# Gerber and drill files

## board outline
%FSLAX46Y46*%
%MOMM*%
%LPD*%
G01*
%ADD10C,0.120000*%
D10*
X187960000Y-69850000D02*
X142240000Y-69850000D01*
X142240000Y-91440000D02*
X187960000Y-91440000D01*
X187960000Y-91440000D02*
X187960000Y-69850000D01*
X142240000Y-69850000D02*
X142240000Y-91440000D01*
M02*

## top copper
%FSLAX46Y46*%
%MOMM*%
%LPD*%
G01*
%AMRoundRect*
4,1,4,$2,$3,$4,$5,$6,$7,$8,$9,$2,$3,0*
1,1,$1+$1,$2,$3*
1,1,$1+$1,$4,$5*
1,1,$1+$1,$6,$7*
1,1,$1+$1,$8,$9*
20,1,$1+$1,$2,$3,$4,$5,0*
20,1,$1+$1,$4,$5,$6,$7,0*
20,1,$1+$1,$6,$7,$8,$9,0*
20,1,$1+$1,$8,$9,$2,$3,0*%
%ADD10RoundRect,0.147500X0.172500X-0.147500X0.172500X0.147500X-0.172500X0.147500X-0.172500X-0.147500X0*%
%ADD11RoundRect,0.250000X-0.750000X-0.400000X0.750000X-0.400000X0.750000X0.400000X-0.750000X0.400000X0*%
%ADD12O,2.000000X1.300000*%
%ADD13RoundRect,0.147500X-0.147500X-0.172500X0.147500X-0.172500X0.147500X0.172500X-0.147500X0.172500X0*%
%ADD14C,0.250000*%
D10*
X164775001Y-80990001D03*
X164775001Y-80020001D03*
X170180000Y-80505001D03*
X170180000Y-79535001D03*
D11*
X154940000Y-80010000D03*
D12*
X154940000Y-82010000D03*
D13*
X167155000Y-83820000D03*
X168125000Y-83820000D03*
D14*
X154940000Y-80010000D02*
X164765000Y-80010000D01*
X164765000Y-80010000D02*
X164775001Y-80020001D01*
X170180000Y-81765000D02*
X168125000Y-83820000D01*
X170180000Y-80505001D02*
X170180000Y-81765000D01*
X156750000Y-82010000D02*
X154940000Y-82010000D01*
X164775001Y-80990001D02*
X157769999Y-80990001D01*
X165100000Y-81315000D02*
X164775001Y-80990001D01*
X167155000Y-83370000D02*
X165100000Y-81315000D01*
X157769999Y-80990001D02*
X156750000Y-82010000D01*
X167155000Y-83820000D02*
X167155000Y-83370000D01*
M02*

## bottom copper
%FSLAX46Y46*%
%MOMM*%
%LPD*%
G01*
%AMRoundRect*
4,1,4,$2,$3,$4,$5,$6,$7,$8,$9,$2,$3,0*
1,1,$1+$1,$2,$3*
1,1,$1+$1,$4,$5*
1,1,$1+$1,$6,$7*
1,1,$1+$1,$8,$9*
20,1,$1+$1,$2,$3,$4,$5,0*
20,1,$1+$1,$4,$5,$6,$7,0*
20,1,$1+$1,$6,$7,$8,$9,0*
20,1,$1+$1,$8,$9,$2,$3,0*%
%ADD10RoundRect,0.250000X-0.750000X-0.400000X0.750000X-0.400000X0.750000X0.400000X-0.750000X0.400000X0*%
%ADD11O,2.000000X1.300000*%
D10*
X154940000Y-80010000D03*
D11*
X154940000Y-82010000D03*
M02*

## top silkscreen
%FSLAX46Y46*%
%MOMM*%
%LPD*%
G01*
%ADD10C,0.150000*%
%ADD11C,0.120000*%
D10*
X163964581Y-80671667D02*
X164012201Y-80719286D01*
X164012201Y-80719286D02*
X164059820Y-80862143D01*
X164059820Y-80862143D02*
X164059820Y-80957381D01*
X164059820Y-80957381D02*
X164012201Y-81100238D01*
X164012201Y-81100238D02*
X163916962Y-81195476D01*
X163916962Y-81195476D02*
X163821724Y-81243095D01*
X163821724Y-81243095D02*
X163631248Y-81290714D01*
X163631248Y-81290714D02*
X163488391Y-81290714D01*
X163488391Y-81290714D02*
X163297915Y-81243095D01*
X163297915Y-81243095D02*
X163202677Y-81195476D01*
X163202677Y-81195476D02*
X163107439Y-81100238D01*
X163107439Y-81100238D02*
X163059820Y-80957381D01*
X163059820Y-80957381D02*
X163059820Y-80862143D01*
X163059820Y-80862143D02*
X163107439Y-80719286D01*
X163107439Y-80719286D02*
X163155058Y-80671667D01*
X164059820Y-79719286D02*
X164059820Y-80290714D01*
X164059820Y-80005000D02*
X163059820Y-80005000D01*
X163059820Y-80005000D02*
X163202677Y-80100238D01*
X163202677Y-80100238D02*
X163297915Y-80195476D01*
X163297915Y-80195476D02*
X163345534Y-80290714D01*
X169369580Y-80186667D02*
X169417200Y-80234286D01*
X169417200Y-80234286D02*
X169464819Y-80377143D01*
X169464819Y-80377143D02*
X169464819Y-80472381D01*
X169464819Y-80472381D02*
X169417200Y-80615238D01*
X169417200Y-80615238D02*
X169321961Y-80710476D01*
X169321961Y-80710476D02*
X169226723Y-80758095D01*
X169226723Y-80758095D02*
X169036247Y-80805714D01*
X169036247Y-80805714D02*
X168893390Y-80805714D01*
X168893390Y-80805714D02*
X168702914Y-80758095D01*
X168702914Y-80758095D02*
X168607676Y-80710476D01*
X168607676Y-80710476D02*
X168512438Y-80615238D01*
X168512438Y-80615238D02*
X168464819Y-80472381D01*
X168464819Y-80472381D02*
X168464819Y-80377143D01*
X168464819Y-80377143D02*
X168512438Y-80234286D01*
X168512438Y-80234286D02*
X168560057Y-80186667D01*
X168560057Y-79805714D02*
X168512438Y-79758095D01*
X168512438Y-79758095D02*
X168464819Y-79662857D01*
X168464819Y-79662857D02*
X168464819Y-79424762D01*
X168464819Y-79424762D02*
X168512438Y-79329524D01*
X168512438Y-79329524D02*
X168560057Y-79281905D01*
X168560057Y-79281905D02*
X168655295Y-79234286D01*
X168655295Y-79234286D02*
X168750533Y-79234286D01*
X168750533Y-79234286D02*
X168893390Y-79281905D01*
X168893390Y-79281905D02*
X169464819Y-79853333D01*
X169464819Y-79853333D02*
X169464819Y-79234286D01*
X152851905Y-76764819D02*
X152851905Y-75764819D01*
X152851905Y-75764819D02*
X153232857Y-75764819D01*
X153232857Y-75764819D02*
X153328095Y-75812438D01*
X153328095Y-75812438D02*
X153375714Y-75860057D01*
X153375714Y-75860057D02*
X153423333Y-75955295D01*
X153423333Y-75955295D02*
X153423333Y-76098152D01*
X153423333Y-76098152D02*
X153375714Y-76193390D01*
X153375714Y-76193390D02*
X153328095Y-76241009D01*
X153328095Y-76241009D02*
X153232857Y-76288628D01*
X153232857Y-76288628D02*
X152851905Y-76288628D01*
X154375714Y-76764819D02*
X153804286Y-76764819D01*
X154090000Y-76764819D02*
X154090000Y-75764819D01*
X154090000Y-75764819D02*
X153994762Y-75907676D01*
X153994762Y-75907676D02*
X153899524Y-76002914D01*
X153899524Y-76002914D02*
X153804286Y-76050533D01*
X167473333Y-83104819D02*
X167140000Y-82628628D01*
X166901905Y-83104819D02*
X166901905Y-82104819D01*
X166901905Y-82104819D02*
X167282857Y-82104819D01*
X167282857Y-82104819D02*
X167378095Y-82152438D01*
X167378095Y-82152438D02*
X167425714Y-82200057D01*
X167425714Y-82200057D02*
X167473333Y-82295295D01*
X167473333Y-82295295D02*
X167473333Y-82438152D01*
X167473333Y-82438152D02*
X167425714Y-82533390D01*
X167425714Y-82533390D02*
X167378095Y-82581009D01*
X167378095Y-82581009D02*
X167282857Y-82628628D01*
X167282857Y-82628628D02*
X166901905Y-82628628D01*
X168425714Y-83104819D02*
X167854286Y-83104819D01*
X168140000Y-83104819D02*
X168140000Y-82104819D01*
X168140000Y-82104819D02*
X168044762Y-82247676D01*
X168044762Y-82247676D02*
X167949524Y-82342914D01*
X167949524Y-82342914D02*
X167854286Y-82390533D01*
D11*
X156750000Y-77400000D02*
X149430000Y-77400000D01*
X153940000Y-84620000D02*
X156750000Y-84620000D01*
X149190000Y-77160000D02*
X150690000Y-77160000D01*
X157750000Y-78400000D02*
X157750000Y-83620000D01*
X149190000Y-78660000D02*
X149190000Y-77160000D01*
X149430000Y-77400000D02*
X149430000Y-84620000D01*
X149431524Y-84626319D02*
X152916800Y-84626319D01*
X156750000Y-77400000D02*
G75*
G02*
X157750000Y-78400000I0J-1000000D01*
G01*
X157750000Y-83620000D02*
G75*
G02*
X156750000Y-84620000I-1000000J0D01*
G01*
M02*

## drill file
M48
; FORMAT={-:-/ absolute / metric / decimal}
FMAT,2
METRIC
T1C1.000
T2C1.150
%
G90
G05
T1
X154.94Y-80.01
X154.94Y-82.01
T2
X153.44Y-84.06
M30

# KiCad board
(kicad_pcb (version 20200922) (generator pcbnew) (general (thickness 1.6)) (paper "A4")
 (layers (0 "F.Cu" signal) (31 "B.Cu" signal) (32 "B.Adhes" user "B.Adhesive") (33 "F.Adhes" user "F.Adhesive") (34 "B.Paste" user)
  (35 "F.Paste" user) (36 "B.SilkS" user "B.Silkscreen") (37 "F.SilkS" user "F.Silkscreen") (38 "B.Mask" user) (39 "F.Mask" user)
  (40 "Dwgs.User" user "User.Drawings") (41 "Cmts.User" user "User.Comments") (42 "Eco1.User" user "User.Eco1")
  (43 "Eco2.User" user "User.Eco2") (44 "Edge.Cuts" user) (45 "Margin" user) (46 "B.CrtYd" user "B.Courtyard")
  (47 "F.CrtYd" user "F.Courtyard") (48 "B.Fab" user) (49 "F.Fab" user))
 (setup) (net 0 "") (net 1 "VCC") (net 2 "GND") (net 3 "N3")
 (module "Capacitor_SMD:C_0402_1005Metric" (layer "F.Cu") (at 164.775001 80.505001 90)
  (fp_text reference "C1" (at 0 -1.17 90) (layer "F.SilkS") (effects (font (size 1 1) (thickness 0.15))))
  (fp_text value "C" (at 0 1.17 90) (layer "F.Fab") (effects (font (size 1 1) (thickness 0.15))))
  (pad "1" smd roundrect (at -0.485 0 90) (size 0.59 0.64) (layers "F.Cu" "F.Paste" "F.Mask") (roundrect_rratio 0.25) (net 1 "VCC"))
  (pad "2" smd roundrect (at 0.485 0 90) (size 0.59 0.64) (layers "F.Cu" "F.Paste" "F.Mask") (roundrect_rratio 0.25) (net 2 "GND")))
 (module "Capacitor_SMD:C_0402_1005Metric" (layer "F.Cu") (at 170.18 80.020001 90)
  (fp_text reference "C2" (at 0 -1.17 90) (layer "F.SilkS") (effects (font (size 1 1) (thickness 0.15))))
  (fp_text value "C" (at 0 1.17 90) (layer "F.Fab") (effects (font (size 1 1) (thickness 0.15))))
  (pad "1" smd roundrect (at -0.485 0 90) (size 0.59 0.64) (layers "F.Cu" "F.Paste" "F.Mask") (roundrect_rratio 0.25) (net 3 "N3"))
  (pad "2" smd roundrect (at 0.485 0 90) (size 0.59 0.64) (layers "F.Cu" "F.Paste" "F.Mask") (roundrect_rratio 0.25) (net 2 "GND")))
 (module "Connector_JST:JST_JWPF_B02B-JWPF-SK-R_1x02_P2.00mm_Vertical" (layer "F.Cu") (at 154.94 80.01)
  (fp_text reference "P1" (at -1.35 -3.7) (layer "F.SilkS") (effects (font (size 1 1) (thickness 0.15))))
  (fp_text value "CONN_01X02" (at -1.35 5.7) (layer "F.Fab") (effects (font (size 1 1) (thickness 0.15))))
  (fp_line (start 1.81 -2.61) (end -5.51 -2.61) (layer "F.SilkS") (width 0.12))
  (fp_line (start -1 4.61) (end 1.81 4.61) (layer "F.SilkS") (width 0.12))
  (fp_line (start -5.75 -2.85) (end -4.25 -2.85) (layer "F.SilkS") (width 0.12))
  (fp_line (start 2.81 -1.61) (end 2.81 3.61) (layer "F.SilkS") (width 0.12))
  (fp_line (start -5.75 -1.35) (end -5.75 -2.85) (layer "F.SilkS") (width 0.12))
  (fp_line (start -5.51 -2.61) (end -5.51 4.61) (layer "F.SilkS") (width 0.12))
  (fp_line (start -5.508476 4.616319) (end -2.0232 4.616319) (layer "F.SilkS") (width 0.12))
  (fp_arc (start 1.81 -1.61) (end 1.81 -2.61) (angle 90) (layer "F.SilkS") (width 0.12))
  (fp_arc (start 1.81 3.61) (end 2.81 3.61) (angle 90) (layer "F.SilkS") (width 0.12))
  (pad "" np_thru_hole circle (at -1.5 4.05) (size 1.15 1.15) (drill 1.15) (layers *.Cu *.Mask))
  (pad "1" thru_hole roundrect (at 0 0) (size 2 1.3) (drill 1) (layers *.Cu *.Mask) (roundrect_rratio 0.192308) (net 2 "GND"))
  (pad "2" thru_hole oval (at 0 2) (size 2 1.3) (drill 1) (layers *.Cu *.Mask) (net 1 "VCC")))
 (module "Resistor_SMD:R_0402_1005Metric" (layer "F.Cu") (at 167.64 83.82)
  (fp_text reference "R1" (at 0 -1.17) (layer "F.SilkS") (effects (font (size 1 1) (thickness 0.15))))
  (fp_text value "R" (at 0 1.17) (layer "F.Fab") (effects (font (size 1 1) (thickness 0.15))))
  (pad "1" smd roundrect (at -0.485 0) (size 0.59 0.64) (layers "F.Cu" "F.Paste" "F.Mask") (roundrect_rratio 0.25) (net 1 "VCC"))
  (pad "2" smd roundrect (at 0.485 0) (size 0.59 0.64) (layers "F.Cu" "F.Paste" "F.Mask") (roundrect_rratio 0.25) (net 3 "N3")))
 (gr_line (start 187.96 69.85) (end 142.24 69.85) (layer "Edge.Cuts") (width 0.12))
 (gr_line (start 142.24 91.44) (end 187.96 91.44) (layer "Edge.Cuts") (width 0.12))
 (gr_line (start 187.96 91.44) (end 187.96 69.85) (layer "Edge.Cuts") (width 0.12))
 (gr_line (start 142.24 69.85) (end 142.24 91.44) (layer "Edge.Cuts") (width 0.12))
 (segment (start 154.94 80.01) (end 164.765 80.01) (width 0.25) (layer "F.Cu") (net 2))
 (segment (start 164.765 80.01) (end 164.775001 80.020001) (width 0.25) (layer "F.Cu") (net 2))
 (segment (start 170.18 81.765) (end 168.125 83.82) (width 0.25) (layer "F.Cu") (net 3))
 (segment (start 170.18 80.505001) (end 170.18 81.765) (width 0.25) (layer "F.Cu") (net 3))
 (segment (start 156.75 82.01) (end 154.94 82.01) (width 0.25) (layer "F.Cu") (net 1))
 (segment (start 164.775001 80.990001) (end 157.769999 80.990001) (width 0.25) (layer "F.Cu") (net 1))
 (segment (start 165.1 81.315) (end 164.775001 80.990001) (width 0.25) (layer "F.Cu") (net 1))
 (segment (start 167.155 83.37) (end 165.1 81.315) (width 0.25) (layer "F.Cu") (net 1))
 (segment (start 157.769999 80.990001) (end 156.75 82.01) (width 0.25) (layer "F.Cu") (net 1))
 (segment (start 167.155 83.82) (end 167.155 83.37) (width 0.25) (layer "F.Cu") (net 1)))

